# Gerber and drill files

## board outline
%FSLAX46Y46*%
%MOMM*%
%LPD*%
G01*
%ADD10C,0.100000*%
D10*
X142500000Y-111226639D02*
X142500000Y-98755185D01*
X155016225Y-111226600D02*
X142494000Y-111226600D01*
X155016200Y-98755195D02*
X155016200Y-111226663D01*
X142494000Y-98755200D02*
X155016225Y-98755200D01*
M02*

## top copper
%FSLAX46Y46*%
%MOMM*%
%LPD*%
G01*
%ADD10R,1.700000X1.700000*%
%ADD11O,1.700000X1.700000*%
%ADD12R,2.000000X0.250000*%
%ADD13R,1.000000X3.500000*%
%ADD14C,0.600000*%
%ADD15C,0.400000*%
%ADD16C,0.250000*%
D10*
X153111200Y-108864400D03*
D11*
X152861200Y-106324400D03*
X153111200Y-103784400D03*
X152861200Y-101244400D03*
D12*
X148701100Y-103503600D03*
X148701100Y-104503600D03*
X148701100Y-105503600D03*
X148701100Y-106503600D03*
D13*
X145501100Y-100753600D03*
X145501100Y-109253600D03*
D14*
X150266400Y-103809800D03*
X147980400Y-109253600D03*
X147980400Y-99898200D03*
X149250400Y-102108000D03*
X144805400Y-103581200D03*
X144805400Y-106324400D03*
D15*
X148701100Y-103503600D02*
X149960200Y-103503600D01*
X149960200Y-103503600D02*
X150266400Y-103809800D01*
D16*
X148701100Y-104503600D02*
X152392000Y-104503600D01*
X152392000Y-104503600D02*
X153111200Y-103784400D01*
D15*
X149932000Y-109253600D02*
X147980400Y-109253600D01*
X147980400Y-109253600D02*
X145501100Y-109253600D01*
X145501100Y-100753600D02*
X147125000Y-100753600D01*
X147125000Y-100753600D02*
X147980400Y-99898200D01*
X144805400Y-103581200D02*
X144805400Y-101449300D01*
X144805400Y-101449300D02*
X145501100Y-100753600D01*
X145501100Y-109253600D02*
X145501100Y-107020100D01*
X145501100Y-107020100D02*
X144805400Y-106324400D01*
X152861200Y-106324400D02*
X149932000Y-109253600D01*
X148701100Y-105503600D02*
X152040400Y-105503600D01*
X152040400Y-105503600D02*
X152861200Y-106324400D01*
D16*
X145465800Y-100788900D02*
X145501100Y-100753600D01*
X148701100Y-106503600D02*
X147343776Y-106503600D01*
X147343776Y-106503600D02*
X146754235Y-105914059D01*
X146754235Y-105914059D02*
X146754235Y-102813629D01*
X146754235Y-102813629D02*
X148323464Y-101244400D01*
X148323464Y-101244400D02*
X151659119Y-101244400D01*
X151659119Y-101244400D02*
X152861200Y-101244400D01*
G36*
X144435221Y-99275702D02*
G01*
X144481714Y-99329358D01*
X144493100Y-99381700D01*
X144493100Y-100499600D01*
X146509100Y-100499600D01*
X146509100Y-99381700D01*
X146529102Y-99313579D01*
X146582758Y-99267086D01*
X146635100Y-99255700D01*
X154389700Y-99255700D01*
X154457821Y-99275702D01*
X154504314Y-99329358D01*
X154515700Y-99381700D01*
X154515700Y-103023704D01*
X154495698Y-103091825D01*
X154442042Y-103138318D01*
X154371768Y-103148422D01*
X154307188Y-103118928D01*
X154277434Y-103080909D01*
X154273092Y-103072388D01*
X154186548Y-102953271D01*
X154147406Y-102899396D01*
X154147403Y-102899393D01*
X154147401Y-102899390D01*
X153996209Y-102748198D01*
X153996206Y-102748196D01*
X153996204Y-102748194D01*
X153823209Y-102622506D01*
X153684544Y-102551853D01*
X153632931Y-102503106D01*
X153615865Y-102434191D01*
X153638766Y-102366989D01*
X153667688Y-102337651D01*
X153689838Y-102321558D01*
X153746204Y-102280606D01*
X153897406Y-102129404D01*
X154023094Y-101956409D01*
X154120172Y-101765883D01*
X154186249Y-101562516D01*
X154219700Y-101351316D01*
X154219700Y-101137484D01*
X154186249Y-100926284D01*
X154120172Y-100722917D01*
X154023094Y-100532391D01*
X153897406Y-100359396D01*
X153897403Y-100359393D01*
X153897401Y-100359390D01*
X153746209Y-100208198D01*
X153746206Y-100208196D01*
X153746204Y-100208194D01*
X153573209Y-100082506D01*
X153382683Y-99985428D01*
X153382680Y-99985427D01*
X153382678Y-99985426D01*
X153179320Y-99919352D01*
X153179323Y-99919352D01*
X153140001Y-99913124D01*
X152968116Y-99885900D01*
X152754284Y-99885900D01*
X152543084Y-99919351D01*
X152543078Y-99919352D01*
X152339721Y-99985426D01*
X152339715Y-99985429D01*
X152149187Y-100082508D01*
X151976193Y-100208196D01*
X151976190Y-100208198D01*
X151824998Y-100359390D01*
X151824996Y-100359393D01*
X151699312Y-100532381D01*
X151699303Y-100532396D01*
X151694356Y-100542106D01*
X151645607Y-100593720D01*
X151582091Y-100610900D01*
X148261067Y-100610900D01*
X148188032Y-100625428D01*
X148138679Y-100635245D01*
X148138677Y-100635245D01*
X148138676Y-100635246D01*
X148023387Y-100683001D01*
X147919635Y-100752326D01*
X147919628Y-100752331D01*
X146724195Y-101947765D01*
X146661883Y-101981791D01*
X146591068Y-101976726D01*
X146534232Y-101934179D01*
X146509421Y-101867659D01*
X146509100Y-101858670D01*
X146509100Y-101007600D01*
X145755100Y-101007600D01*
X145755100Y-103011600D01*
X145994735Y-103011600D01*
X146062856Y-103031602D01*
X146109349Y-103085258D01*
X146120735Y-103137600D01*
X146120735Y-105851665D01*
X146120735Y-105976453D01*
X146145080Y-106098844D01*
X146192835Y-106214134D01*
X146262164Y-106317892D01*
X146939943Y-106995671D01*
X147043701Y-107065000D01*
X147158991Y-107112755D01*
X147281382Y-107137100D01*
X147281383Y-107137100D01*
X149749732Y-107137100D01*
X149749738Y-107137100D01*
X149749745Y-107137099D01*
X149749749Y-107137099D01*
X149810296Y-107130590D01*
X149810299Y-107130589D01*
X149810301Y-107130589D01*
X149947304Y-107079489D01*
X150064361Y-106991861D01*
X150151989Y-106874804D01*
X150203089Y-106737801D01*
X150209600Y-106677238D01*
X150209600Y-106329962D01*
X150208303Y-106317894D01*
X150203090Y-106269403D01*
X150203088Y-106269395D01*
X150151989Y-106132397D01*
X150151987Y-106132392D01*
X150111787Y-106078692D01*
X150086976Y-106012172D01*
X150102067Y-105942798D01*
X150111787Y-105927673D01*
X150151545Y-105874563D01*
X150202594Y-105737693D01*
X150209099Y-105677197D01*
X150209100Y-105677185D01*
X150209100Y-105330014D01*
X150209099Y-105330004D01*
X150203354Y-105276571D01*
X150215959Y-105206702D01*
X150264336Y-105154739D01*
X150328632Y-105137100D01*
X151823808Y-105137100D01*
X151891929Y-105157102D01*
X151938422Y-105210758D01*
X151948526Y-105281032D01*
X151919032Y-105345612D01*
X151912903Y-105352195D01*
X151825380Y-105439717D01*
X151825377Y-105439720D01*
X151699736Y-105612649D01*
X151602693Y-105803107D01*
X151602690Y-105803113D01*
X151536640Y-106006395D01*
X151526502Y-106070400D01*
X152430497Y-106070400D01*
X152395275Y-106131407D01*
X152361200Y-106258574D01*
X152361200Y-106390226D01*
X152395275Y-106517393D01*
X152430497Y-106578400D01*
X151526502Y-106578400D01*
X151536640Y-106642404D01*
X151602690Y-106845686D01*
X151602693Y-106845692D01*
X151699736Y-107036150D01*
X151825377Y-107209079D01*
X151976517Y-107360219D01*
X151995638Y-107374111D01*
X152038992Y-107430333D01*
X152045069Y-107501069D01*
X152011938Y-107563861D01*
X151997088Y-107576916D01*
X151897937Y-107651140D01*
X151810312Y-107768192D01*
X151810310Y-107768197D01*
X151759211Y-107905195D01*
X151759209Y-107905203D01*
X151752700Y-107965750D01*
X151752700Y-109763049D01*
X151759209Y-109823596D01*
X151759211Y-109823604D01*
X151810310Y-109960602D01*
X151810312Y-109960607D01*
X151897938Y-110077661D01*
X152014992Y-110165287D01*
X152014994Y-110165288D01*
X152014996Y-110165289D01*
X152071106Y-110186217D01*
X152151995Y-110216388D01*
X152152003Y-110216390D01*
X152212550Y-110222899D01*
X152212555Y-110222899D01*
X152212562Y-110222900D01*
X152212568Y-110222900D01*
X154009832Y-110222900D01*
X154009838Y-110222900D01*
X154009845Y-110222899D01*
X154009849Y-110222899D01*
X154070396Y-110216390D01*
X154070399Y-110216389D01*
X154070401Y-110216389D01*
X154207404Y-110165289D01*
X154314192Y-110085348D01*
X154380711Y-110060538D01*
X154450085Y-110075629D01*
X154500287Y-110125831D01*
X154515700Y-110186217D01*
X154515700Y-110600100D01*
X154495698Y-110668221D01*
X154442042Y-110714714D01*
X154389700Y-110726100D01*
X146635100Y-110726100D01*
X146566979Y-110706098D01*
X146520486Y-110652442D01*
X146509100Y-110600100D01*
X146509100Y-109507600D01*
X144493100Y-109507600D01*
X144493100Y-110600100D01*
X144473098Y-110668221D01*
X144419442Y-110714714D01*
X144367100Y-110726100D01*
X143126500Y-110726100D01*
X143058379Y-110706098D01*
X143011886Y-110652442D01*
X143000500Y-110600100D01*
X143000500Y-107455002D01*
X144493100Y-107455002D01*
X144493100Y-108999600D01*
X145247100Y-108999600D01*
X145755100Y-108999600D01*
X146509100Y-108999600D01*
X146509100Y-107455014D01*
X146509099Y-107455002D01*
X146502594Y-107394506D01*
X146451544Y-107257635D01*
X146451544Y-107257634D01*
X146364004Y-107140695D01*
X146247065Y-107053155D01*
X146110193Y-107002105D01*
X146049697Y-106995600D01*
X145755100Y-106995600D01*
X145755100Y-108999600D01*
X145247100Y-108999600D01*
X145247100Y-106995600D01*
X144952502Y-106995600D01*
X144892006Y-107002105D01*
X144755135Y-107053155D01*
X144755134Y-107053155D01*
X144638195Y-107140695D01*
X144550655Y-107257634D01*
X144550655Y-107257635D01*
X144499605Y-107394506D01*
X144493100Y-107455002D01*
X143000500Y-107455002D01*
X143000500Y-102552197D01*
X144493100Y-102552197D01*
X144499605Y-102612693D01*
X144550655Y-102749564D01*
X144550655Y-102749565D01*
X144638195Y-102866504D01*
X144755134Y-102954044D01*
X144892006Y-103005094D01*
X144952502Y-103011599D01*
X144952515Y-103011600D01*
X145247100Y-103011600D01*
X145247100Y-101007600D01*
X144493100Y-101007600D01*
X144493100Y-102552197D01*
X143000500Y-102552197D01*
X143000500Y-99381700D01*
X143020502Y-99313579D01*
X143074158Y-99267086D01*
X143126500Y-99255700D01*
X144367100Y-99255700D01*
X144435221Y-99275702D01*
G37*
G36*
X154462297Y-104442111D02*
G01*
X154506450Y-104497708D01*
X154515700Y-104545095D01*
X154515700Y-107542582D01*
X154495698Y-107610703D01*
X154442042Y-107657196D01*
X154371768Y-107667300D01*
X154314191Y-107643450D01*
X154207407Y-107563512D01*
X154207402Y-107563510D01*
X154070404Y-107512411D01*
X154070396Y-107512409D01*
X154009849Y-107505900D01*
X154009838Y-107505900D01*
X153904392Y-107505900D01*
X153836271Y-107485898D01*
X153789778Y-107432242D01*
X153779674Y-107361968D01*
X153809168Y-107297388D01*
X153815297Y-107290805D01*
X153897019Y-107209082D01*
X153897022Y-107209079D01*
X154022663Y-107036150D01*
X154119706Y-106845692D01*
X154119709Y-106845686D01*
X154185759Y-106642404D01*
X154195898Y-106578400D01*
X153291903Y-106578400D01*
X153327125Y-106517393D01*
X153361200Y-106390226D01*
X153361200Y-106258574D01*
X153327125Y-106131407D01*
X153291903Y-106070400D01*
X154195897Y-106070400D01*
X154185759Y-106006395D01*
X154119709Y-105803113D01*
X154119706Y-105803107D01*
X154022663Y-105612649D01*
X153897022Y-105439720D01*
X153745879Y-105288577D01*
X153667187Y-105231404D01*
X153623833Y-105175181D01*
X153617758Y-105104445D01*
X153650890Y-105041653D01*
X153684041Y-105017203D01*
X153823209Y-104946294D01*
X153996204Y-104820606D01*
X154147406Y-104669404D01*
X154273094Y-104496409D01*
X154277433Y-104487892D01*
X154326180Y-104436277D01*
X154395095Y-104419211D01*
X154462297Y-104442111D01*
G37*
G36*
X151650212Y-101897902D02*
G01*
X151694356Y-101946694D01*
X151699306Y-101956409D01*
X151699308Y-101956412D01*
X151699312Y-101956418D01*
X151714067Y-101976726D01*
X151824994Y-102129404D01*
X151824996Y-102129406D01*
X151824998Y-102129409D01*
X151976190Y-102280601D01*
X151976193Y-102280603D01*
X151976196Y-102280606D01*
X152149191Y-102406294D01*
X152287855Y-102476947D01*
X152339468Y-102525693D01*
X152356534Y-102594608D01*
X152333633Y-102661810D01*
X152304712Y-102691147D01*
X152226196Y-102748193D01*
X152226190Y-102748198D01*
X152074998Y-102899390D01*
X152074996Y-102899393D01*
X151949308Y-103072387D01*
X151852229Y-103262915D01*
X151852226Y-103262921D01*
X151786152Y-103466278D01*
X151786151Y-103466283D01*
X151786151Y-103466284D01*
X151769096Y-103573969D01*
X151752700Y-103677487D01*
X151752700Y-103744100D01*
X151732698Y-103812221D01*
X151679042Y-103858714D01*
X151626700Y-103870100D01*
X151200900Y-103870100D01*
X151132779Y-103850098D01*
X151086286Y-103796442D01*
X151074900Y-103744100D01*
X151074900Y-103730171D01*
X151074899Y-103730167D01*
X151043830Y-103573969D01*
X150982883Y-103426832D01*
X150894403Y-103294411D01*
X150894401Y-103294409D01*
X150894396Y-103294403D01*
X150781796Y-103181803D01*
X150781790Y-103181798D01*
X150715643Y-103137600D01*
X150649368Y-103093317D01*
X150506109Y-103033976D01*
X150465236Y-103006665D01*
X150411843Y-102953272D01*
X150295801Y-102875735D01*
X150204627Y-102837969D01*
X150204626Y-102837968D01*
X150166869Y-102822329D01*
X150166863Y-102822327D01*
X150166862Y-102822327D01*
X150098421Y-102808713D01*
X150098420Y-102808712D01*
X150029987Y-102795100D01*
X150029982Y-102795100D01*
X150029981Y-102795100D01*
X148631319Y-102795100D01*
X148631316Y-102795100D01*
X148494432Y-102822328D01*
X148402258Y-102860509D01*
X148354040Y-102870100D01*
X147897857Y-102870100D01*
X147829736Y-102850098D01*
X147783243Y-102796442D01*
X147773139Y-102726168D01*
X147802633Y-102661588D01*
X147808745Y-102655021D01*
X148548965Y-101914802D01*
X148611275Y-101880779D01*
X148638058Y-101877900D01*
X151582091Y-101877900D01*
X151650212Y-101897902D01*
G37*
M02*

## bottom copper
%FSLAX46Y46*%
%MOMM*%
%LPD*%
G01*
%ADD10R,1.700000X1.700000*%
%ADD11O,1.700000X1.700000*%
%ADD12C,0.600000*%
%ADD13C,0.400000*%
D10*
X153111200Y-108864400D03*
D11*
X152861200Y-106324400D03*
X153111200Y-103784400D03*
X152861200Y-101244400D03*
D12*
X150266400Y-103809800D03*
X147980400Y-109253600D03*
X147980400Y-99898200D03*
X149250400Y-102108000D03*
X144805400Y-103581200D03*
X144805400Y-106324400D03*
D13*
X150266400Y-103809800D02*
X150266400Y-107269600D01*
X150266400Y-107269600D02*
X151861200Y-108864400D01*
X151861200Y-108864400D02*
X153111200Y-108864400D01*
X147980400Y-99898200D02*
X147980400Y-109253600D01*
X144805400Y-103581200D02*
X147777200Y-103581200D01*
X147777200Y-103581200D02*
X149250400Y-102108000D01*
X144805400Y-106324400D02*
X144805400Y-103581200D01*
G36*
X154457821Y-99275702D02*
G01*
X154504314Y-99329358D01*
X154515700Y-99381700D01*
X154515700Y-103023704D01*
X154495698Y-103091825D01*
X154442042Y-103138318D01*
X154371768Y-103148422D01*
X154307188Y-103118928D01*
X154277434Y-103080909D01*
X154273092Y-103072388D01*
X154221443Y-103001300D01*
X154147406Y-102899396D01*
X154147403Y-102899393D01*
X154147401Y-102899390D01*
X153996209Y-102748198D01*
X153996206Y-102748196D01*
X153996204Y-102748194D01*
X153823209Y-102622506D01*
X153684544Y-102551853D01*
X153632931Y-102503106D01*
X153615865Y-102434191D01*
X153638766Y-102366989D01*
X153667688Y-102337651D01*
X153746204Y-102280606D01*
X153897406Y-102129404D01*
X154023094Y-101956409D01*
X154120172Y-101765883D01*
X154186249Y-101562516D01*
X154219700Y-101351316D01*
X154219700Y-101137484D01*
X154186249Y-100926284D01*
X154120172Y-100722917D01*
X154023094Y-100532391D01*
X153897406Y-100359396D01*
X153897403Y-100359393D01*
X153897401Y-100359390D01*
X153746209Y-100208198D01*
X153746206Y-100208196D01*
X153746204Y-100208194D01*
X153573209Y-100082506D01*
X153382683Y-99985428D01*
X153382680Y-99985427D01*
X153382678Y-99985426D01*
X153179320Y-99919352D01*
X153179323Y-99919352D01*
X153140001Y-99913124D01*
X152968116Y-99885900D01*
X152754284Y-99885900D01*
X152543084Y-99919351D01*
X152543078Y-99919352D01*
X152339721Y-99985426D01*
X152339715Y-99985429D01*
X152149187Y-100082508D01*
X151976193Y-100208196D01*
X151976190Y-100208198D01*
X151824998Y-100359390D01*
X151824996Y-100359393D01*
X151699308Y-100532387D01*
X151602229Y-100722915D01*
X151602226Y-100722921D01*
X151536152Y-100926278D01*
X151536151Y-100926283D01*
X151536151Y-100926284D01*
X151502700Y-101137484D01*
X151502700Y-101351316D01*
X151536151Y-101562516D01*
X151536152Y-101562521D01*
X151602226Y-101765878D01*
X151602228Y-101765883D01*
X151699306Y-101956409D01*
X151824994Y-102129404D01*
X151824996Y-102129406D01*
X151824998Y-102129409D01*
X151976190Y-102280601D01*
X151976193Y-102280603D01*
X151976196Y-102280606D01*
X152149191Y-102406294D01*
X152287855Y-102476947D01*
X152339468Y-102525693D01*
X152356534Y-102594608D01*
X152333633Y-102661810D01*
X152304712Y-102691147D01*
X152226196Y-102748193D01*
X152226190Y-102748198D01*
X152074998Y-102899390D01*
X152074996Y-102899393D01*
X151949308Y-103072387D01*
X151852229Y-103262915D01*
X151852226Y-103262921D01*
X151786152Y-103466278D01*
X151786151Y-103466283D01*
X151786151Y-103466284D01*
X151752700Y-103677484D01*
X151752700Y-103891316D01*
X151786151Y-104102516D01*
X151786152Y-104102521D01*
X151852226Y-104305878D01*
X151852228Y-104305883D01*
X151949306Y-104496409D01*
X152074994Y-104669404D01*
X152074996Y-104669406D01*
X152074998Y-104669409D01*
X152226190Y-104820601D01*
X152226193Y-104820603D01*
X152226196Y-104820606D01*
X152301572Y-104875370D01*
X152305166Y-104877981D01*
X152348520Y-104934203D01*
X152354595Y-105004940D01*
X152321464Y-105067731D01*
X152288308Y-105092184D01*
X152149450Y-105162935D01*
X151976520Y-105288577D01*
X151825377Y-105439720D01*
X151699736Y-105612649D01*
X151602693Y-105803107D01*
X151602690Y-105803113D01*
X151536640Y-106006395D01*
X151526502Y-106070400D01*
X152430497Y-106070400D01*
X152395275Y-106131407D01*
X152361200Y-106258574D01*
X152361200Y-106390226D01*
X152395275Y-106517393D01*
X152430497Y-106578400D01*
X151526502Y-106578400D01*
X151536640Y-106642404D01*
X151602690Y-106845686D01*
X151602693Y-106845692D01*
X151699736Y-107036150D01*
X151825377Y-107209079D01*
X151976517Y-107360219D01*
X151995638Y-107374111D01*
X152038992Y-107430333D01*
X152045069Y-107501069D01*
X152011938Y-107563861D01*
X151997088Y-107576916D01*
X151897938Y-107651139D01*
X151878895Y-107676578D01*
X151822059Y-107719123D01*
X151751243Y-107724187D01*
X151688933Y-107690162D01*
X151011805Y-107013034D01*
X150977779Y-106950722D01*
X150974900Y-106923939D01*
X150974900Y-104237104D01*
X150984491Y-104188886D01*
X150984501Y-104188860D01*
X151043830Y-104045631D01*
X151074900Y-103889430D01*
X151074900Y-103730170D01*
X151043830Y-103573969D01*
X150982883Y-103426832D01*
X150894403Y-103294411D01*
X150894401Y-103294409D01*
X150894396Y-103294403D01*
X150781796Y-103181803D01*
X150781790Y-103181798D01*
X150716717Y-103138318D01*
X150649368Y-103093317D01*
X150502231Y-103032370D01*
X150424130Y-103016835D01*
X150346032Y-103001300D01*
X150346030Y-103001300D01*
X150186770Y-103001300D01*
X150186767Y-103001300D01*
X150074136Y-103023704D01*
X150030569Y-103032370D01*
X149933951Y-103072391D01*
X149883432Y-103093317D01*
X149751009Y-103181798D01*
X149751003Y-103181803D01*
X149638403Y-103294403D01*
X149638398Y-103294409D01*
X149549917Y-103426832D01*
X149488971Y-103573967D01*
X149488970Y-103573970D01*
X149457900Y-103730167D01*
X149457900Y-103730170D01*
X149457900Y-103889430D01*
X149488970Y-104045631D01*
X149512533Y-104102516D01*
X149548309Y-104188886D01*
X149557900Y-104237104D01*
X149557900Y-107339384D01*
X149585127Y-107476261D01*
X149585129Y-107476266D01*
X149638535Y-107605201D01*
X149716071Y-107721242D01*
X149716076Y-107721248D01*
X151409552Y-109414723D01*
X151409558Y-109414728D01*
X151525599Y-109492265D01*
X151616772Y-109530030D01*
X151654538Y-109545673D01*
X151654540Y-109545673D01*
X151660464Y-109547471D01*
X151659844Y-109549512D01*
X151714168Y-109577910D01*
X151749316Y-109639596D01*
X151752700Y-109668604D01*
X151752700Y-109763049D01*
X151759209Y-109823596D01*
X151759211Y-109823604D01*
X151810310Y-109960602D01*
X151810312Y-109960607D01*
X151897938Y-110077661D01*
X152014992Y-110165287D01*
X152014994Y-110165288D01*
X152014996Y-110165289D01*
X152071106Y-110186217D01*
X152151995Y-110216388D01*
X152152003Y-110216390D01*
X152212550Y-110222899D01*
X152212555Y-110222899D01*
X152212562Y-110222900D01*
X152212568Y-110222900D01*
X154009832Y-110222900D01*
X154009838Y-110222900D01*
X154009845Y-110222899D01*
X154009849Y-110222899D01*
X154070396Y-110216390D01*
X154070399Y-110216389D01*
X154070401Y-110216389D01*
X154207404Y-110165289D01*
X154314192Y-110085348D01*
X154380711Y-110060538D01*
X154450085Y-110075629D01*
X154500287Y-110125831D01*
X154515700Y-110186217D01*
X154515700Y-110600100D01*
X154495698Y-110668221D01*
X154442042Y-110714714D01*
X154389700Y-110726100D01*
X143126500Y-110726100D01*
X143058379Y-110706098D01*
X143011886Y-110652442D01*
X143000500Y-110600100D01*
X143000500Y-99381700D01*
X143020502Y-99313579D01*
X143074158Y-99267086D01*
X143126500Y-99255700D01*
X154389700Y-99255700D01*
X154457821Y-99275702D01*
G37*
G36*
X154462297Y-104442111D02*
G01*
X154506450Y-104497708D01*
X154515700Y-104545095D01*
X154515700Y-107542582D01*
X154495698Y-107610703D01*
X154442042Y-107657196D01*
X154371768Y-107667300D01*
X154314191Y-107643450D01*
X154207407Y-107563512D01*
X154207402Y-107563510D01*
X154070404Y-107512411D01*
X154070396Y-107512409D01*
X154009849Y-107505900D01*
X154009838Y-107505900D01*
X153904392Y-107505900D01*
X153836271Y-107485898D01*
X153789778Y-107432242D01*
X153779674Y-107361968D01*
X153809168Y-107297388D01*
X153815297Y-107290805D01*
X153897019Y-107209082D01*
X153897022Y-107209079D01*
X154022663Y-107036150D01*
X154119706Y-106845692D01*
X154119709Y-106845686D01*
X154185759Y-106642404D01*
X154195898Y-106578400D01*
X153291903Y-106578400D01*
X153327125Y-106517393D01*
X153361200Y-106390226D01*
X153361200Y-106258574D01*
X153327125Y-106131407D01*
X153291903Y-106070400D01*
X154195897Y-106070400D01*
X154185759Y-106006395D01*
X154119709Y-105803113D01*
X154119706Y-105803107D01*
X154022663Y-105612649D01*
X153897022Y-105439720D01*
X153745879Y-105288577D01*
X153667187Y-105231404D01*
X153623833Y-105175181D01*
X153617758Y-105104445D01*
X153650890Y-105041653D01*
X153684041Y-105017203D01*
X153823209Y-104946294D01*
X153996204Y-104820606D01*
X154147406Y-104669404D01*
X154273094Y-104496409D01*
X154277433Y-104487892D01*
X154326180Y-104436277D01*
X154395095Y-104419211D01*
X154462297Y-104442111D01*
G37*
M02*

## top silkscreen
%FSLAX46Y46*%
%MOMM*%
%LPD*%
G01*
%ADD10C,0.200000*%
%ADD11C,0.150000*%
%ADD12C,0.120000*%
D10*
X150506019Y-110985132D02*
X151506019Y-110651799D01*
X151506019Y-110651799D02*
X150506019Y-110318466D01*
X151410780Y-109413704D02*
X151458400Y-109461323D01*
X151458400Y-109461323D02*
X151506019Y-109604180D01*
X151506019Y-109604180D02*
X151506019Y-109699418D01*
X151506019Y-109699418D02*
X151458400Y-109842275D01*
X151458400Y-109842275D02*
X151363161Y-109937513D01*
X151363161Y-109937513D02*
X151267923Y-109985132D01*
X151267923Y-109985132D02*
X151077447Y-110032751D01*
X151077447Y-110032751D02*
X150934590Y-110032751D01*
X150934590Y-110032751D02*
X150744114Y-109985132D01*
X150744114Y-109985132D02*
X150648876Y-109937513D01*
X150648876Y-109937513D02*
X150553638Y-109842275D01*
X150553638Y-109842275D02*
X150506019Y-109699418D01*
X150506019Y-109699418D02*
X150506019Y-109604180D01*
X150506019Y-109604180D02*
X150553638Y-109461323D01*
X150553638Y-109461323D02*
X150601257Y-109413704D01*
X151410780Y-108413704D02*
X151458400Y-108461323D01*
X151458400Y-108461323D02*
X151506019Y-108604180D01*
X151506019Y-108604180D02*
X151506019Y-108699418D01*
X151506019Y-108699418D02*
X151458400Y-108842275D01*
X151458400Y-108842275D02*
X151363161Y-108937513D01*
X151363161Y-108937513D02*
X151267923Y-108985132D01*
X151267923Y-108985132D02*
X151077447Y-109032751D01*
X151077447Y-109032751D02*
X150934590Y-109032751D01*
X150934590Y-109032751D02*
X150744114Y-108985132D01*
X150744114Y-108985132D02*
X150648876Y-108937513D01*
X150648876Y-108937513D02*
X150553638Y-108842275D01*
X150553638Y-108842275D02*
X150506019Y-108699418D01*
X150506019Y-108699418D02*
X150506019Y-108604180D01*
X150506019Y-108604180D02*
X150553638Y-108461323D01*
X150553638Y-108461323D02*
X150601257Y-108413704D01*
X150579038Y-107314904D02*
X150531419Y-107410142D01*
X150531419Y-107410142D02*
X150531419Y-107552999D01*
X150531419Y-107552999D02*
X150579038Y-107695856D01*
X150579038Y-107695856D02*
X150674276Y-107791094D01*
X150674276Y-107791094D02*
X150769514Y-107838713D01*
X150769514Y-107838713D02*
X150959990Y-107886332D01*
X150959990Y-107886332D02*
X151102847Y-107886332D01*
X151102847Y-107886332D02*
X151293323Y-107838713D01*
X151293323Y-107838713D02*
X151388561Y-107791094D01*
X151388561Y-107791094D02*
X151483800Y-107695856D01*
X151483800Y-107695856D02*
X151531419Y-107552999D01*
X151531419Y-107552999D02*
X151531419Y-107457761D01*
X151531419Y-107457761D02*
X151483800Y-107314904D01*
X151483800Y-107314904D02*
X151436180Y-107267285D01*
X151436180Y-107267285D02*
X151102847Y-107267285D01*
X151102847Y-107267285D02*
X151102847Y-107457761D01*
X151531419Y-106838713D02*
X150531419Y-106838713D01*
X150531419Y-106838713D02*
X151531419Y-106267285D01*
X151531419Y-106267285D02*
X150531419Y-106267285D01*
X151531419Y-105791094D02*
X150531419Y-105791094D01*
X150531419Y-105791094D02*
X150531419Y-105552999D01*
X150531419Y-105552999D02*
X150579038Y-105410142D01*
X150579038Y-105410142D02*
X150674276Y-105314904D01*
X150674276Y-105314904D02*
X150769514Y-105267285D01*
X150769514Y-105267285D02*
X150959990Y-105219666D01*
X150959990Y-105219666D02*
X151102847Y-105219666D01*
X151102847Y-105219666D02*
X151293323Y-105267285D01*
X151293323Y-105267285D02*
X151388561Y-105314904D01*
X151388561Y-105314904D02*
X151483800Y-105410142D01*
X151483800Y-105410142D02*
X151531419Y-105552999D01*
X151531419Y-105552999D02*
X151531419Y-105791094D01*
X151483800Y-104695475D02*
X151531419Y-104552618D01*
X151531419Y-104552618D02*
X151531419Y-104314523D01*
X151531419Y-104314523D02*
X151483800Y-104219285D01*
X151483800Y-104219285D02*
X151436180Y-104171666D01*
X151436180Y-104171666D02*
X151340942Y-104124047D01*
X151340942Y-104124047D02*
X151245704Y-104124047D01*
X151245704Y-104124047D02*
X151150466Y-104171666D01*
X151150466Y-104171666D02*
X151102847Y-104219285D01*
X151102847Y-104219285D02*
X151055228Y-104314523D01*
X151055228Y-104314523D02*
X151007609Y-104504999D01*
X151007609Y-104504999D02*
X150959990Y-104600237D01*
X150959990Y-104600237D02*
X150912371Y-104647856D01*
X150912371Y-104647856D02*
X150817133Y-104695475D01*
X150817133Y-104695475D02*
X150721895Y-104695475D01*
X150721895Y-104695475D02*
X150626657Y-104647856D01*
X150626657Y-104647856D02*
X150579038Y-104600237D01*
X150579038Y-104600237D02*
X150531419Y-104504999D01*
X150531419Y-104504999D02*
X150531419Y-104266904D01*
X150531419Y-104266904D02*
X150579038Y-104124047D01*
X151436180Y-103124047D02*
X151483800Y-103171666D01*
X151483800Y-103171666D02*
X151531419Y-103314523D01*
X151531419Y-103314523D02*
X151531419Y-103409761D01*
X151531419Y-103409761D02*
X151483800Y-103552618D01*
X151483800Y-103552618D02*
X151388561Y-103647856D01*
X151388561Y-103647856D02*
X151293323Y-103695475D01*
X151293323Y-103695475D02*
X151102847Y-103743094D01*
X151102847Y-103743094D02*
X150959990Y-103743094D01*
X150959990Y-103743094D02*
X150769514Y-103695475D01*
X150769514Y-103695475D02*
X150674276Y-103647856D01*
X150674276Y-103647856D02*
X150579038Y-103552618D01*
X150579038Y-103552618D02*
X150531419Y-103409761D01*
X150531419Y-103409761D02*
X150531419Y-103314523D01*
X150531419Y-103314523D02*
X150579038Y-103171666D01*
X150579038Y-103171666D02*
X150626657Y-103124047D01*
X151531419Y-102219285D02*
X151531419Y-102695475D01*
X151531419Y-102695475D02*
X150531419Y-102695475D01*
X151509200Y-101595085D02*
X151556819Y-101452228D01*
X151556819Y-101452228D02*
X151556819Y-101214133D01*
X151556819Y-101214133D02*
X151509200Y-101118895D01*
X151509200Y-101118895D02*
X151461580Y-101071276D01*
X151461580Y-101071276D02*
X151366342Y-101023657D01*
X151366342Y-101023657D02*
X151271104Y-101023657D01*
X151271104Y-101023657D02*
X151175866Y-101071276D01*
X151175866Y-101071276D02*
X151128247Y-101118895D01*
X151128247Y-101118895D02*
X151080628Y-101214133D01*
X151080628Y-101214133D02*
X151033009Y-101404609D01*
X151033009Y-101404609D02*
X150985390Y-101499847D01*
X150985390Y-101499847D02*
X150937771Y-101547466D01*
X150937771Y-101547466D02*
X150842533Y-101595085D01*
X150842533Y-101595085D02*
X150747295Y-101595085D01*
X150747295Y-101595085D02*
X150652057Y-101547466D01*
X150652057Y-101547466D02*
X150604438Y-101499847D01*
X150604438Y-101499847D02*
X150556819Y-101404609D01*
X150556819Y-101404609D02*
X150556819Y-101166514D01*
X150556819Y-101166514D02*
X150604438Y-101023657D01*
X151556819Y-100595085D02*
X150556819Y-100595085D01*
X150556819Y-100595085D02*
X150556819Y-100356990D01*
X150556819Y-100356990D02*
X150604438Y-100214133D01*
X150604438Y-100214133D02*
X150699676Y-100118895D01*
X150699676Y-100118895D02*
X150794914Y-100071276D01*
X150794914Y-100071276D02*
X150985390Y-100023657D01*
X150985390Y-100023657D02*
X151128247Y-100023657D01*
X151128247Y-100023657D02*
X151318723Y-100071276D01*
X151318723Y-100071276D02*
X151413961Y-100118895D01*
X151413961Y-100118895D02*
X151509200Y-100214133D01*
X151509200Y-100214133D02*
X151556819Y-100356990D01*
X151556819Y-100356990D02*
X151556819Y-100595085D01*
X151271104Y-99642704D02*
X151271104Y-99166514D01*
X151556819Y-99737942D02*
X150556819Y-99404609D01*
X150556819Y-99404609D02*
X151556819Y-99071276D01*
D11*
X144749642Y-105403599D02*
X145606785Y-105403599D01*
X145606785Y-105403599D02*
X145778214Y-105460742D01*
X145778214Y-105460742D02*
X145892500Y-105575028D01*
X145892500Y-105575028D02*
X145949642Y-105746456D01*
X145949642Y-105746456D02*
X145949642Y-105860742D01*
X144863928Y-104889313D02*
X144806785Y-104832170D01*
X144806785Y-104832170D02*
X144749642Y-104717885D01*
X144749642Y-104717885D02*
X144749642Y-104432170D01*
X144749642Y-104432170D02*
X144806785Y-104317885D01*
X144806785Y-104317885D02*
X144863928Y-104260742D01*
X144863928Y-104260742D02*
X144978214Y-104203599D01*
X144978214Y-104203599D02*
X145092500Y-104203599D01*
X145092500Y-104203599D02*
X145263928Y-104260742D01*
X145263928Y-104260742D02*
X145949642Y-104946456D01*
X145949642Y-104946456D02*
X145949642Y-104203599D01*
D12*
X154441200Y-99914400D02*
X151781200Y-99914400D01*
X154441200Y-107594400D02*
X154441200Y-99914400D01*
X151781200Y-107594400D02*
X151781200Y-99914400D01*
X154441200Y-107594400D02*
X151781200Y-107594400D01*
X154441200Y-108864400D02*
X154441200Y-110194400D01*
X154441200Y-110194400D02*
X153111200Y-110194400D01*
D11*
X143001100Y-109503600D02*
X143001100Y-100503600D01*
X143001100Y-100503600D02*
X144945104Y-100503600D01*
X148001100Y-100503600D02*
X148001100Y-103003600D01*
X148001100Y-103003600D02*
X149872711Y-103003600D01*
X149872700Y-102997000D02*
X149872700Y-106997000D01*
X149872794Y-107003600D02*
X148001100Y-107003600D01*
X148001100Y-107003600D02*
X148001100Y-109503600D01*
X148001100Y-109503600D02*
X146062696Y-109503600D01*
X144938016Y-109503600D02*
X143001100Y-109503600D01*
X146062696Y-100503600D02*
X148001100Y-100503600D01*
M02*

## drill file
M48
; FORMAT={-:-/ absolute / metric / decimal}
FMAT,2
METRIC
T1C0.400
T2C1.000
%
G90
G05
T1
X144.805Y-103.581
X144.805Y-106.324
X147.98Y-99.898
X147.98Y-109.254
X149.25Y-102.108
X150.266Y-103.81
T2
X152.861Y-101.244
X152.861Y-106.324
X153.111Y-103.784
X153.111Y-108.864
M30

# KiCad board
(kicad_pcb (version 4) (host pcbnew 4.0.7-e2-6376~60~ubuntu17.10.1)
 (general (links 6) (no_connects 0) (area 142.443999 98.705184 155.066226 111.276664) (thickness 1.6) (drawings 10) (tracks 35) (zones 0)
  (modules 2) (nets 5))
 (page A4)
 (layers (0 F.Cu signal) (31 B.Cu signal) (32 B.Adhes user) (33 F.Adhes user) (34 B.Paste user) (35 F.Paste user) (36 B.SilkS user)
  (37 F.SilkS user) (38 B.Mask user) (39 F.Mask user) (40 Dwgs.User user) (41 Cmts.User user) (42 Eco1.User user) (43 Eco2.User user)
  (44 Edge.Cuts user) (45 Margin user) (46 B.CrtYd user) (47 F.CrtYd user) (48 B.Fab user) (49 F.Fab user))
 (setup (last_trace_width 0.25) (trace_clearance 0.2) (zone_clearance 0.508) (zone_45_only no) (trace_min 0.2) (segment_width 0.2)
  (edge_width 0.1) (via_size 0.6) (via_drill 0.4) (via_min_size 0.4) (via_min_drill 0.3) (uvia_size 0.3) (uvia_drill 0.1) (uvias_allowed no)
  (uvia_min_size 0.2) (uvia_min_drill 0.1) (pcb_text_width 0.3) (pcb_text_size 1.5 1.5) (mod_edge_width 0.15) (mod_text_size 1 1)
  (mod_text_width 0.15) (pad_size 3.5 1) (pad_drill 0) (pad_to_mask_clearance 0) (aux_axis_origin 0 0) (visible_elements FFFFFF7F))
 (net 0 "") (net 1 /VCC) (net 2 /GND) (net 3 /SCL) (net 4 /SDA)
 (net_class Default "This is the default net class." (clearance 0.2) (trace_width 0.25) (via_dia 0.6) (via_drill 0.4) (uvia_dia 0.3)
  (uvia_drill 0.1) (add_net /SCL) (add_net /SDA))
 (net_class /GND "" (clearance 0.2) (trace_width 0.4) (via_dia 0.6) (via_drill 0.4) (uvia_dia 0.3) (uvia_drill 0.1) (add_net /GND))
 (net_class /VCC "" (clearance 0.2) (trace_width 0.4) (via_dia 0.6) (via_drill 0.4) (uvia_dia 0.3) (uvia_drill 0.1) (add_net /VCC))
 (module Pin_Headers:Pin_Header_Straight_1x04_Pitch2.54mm (layer F.Cu) (at 153.1112 108.8644 180)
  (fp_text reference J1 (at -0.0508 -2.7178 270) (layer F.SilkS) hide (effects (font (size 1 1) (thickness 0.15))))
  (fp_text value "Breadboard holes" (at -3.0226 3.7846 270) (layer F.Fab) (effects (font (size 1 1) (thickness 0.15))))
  (fp_line (start -1.33 8.95) (end 1.33 8.95) (layer F.SilkS) (width 0.12))
  (fp_line (start -1.33 1.27) (end -1.33 8.95) (layer F.SilkS) (width 0.12))
  (fp_line (start 1.33 1.27) (end 1.33 8.95) (layer F.SilkS) (width 0.12))
  (fp_line (start -1.33 1.27) (end 1.33 1.27) (layer F.SilkS) (width 0.12))
  (fp_line (start -1.33 0) (end -1.33 -1.33) (layer F.SilkS) (width 0.12))
  (fp_line (start -1.33 -1.33) (end 0 -1.33) (layer F.SilkS) (width 0.12))
  (pad 1 thru_hole rect (at 0 0 180) (size 1.7 1.7) (drill 1) (layers *.Cu *.Mask) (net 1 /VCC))
  (pad 2 thru_hole oval (at 0.25 2.54 180) (size 1.7 1.7) (drill 1) (layers *.Cu *.Mask) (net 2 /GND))
  (pad 3 thru_hole oval (at 0 5.08 180) (size 1.7 1.7) (drill 1) (layers *.Cu *.Mask) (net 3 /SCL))
  (pad 4 thru_hole oval (at 0.25 7.62 180) (size 1.7 1.7) (drill 1) (layers *.Cu *.Mask) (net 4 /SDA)))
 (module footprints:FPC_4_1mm (layer F.Cu) (at 148.5011 105.0036 270)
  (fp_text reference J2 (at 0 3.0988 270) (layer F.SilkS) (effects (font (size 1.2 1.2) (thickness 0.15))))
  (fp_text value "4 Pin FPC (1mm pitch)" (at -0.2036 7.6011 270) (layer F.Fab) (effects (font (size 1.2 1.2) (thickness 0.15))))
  (fp_line (start 4.5 5.5) (end -4.5 5.5) (layer F.SilkS) (width 0.15))
  (fp_line (start -4.5 5.5) (end -4.5 3.555996) (layer F.SilkS) (width 0.15))
  (fp_line (start -4.5 0.5) (end -2 0.5) (layer F.SilkS) (width 0.15))
  (fp_line (start -2 0.5) (end -2 -1.371611) (layer F.SilkS) (width 0.15))
  (fp_line (start -2.0066 -1.3716) (end 1.9934 -1.3716) (layer F.SilkS) (width 0.15))
  (fp_line (start 2 -1.371694) (end 2 0.5) (layer F.SilkS) (width 0.15))
  (fp_line (start 2 0.5) (end 4.5 0.5) (layer F.SilkS) (width 0.15))
  (fp_line (start 4.5 0.5) (end 4.5 2.438404) (layer F.SilkS) (width 0.15))
  (fp_line (start 4.5 3.563084) (end 4.5 5.5) (layer F.SilkS) (width 0.15))
  (fp_line (start -4.5 2.438404) (end -4.5 0.5) (layer F.SilkS) (width 0.15))
  (pad 1 smd rect (at -1.5 -0.2 270) (size 0.25 2) (layers F.Cu F.Paste F.Mask) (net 1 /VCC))
  (pad 2 smd rect (at -0.5 -0.2 270) (size 0.25 2) (layers F.Cu F.Paste F.Mask) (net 3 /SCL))
  (pad 3 smd rect (at 0.5 -0.2 270) (size 0.25 2) (layers F.Cu F.Paste F.Mask) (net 2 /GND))
  (pad 4 smd rect (at 1.5 -0.2 270) (size 0.25 2) (layers F.Cu F.Paste F.Mask) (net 4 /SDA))
  (pad 0 smd rect (at -4.25 3 270) (size 3.5 1) (layers F.Cu F.Paste F.Mask) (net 2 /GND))
  (pad 0 smd rect (at 4.25 3 270) (size 3.5 1) (layers F.Cu F.Paste F.Mask) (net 2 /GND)))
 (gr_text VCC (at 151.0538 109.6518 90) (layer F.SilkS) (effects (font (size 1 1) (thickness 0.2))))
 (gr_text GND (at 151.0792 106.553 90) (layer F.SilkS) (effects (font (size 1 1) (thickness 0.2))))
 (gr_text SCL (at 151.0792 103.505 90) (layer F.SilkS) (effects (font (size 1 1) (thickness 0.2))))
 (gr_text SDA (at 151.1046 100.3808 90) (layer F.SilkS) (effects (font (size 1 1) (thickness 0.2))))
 (gr_line (start 142.5 111.226639) (end 142.5 98.755185) (angle 90) (layer Edge.Cuts) (width 0.1))
 (gr_line (start 155.016225 111.2266) (end 142.494 111.2266) (angle 90) (layer Edge.Cuts) (width 0.1))
 (gr_line (start 155.0162 98.755195) (end 155.0162 111.226663) (angle 90) (layer Edge.Cuts) (width 0.1))
 (gr_line (start 142.494 98.7552) (end 155.016225 98.7552) (angle 90) (layer Edge.Cuts) (width 0.1))
 (segment (start 150.2664 103.8098) (end 150.2664 107.2696) (width 0.4) (layer B.Cu) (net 1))
 (segment (start 150.2664 107.2696) (end 151.8612 108.8644) (width 0.4) (layer B.Cu) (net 1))
 (segment (start 151.8612 108.8644) (end 153.1112 108.8644) (width 0.4) (layer B.Cu) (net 1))
 (segment (start 148.7011 103.5036) (end 149.9602 103.5036) (width 0.4) (layer F.Cu) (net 1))
 (segment (start 149.9602 103.5036) (end 150.2664 103.8098) (width 0.4) (layer F.Cu) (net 1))
 (via (at 150.2664 103.8098) (size 0.6) (drill 0.4) (layers F.Cu B.Cu) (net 1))
 (segment (start 148.7011 104.5036) (end 152.392 104.5036) (width 0.25) (layer F.Cu) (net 3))
 (segment (start 152.392 104.5036) (end 153.1112 103.7844) (width 0.25) (layer F.Cu) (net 3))
 (segment (start 149.932 109.2536) (end 147.9804 109.2536) (width 0.4) (layer F.Cu) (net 2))
 (segment (start 147.9804 109.2536) (end 145.5011 109.2536) (width 0.4) (layer F.Cu) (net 2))
 (segment (start 147.9804 99.8982) (end 147.9804 109.2536) (width 0.4) (layer B.Cu) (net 2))
 (via (at 147.9804 109.2536) (size 0.6) (drill 0.4) (layers F.Cu B.Cu) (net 2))
 (segment (start 145.5011 100.7536) (end 147.125 100.7536) (width 0.4) (layer F.Cu) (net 2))
 (segment (start 147.125 100.7536) (end 147.9804 99.8982) (width 0.4) (layer F.Cu) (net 2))
 (via (at 147.9804 99.8982) (size 0.6) (drill 0.4) (layers F.Cu B.Cu) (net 2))
 (segment (start 144.8054 103.5812) (end 147.7772 103.5812) (width 0.4) (layer B.Cu) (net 2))
 (segment (start 147.7772 103.5812) (end 149.2504 102.108) (width 0.4) (layer B.Cu) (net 2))
 (via (at 149.2504 102.108) (size 0.6) (drill 0.4) (layers F.Cu B.Cu) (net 2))
 (segment (start 144.8054 103.5812) (end 144.8054 101.4493) (width 0.4) (layer F.Cu) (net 2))
 (segment (start 144.8054 101.4493) (end 145.5011 100.7536) (width 0.4) (layer F.Cu) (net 2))
 (segment (start 144.8054 106.3244) (end 144.8054 103.5812) (width 0.4) (layer B.Cu) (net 2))
 (via (at 144.8054 103.5812) (size 0.6) (drill 0.4) (layers F.Cu B.Cu) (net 2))
 (segment (start 145.5011 109.2536) (end 145.5011 107.0201) (width 0.4) (layer F.Cu) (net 2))
 (segment (start 145.5011 107.0201) (end 144.8054 106.3244) (width 0.4) (layer F.Cu) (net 2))
 (via (at 144.8054 106.3244) (size 0.6) (drill 0.4) (layers F.Cu B.Cu) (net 2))
 (segment (start 152.8612 106.3244) (end 149.932 109.2536) (width 0.4) (layer F.Cu) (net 2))
 (segment (start 148.7011 105.5036) (end 152.0404 105.5036) (width 0.4) (layer F.Cu) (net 2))
 (segment (start 152.0404 105.5036) (end 152.8612 106.3244) (width 0.4) (layer F.Cu) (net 2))
 (segment (start 145.4658 100.7889) (end 145.5011 100.7536) (width 0.25) (layer F.Cu) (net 2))
 (segment (start 148.7011 106.5036) (end 147.343776 106.5036) (width 0.25) (layer F.Cu) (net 4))
 (segment (start 147.343776 106.5036) (end 146.754235 105.914059) (width 0.25) (layer F.Cu) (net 4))
 (segment (start 146.754235 105.914059) (end 146.754235 102.813629) (width 0.25) (layer F.Cu) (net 4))
 (segment (start 146.754235 102.813629) (end 148.323464 101.2444) (width 0.25) (layer F.Cu) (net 4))
 (segment (start 148.323464 101.2444) (end 151.659119 101.2444) (width 0.25) (layer F.Cu) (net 4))
 (segment (start 151.659119 101.2444) (end 152.8612 101.2444) (width 0.25) (layer F.Cu) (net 4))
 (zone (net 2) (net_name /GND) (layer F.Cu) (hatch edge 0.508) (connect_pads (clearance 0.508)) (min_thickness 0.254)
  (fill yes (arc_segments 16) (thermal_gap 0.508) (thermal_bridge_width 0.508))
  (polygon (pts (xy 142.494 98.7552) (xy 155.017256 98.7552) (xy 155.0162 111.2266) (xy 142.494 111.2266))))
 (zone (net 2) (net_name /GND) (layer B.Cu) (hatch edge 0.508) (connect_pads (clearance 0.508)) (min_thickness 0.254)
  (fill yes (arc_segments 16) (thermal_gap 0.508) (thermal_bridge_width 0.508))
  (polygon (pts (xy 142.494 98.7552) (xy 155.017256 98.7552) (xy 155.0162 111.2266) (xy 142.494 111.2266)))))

